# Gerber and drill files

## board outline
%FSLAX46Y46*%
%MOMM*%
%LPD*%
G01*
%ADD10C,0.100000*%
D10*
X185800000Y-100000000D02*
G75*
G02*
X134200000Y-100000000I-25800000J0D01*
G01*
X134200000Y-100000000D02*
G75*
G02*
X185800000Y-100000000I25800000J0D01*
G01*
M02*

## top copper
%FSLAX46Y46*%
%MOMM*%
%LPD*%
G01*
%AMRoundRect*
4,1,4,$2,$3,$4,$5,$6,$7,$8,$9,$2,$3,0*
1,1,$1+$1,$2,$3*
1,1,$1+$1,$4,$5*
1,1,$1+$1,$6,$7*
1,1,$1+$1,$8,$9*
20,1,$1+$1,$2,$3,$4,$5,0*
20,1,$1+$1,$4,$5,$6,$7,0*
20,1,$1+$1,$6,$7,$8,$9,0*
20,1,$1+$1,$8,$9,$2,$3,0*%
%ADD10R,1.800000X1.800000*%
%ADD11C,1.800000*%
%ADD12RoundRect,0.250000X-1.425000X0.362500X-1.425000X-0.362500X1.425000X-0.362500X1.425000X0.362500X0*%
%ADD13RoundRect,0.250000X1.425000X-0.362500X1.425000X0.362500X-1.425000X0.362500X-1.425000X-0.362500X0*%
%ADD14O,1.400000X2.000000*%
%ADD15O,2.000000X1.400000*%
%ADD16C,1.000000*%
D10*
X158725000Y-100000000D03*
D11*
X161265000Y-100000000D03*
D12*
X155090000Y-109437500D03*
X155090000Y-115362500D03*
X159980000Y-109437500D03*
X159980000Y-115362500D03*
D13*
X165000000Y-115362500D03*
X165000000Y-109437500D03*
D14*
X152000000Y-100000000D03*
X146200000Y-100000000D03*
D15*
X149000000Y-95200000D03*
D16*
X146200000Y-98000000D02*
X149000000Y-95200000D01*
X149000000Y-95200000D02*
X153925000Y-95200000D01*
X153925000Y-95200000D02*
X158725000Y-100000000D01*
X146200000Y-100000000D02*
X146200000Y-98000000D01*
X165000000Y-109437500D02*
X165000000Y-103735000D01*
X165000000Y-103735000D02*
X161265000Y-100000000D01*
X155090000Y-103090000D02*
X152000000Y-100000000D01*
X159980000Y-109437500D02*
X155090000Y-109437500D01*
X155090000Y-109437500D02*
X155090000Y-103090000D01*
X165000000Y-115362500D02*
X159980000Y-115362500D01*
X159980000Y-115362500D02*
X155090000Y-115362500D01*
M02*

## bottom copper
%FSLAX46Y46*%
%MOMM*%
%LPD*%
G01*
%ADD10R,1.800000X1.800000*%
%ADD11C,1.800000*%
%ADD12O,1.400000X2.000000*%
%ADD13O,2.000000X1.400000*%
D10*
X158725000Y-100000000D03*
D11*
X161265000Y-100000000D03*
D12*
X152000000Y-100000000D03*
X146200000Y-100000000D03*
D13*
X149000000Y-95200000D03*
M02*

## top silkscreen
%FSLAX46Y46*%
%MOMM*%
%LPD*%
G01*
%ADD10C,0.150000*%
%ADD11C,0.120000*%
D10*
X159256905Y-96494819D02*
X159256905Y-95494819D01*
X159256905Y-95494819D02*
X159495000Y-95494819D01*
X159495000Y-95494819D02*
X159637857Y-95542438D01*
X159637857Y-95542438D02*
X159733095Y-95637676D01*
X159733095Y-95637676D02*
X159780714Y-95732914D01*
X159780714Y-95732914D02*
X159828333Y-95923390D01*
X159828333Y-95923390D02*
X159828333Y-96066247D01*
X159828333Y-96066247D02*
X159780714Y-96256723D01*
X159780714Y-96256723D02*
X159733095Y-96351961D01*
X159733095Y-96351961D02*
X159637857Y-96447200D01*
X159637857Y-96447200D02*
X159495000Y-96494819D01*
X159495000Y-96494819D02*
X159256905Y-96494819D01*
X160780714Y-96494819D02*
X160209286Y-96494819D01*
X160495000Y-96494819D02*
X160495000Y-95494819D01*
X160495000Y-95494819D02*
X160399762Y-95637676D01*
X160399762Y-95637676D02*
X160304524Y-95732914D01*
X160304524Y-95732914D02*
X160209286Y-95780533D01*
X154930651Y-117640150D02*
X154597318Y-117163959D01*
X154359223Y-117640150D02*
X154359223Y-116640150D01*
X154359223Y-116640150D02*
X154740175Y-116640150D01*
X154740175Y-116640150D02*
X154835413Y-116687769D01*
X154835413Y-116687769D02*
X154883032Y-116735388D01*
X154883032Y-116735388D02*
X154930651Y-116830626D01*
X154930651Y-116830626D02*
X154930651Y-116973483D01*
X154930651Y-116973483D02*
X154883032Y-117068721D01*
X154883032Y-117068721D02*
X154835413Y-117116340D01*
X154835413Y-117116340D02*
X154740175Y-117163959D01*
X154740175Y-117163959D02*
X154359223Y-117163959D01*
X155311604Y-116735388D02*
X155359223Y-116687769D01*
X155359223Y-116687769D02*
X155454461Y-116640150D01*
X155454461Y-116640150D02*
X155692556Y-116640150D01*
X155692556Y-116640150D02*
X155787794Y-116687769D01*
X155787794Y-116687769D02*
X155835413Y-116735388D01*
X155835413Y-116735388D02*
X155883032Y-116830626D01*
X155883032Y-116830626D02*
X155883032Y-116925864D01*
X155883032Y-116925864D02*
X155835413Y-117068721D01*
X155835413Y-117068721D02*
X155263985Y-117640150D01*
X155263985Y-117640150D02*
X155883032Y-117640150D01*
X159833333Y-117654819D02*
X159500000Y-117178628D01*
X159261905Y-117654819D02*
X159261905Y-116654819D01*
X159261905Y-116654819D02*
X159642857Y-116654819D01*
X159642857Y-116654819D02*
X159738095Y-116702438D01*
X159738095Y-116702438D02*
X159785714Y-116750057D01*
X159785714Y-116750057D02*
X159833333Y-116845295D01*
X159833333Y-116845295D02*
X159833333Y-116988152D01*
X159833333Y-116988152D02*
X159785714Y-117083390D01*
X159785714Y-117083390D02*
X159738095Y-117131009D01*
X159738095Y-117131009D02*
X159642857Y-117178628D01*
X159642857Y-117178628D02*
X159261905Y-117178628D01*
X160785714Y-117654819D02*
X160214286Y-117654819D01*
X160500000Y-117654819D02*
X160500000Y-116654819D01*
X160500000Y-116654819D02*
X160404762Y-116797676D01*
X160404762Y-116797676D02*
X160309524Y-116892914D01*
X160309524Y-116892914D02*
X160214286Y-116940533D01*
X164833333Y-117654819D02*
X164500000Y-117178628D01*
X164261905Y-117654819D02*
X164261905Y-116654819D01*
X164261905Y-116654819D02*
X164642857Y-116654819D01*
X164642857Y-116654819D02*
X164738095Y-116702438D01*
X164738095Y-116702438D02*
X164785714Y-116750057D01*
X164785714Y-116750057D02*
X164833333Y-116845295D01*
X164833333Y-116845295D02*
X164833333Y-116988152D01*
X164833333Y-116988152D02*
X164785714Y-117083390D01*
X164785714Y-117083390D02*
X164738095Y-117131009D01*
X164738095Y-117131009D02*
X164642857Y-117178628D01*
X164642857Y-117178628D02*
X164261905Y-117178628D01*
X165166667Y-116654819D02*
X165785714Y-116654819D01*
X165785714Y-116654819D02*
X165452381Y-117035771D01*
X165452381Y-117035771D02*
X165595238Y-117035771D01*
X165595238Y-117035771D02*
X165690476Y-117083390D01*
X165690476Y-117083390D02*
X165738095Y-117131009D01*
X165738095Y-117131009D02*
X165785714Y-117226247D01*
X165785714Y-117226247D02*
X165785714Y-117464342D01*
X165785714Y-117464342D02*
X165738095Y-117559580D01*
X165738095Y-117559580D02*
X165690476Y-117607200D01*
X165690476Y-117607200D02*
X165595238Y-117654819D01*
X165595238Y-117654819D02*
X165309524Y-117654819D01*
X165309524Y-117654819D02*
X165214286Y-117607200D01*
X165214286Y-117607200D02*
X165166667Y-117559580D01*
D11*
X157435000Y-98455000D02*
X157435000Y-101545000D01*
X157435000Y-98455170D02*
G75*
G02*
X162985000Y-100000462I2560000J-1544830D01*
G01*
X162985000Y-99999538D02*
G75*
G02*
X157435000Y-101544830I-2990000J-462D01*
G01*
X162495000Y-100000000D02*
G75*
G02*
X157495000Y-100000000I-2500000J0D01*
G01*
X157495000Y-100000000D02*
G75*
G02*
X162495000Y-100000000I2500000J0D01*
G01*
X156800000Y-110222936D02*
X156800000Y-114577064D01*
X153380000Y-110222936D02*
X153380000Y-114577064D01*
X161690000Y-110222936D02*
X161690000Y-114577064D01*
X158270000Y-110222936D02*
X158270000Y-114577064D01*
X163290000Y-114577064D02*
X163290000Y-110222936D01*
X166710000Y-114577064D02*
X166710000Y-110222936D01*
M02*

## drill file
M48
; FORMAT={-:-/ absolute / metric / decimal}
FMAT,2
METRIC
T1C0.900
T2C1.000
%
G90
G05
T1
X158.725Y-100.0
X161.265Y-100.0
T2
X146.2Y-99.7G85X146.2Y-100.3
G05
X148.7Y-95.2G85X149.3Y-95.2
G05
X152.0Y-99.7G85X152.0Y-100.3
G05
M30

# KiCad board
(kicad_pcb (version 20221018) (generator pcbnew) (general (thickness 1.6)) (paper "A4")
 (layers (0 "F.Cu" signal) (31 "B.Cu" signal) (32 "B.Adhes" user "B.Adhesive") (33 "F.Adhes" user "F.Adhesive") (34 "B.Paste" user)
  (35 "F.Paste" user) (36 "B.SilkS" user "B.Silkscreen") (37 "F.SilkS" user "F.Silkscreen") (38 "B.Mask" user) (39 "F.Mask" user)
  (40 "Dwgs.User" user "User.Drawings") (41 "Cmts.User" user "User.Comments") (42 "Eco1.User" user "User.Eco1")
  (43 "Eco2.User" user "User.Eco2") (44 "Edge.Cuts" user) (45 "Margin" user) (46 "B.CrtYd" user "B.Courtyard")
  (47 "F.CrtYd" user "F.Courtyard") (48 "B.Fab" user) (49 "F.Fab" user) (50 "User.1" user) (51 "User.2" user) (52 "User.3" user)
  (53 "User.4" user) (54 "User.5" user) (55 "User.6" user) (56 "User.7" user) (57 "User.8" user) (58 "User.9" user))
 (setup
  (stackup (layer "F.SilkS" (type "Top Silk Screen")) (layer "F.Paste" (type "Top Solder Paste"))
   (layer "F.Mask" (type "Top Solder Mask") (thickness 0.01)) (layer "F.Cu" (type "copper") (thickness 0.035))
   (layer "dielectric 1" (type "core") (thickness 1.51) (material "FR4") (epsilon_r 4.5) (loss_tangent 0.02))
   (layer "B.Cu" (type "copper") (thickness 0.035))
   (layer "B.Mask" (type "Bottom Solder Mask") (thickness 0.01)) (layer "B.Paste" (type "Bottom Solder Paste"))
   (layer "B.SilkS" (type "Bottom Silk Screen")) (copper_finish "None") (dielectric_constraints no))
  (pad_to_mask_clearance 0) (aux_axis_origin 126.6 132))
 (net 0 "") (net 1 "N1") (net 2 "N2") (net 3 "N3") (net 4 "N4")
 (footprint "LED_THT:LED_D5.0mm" (layer "F.Cu") (at 158.725 100)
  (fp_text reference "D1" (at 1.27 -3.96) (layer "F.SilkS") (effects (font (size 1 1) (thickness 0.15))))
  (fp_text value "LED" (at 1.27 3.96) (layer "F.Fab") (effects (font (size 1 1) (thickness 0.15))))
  (fp_line (start -1.29 -1.545) (end -1.29 1.545) (stroke (width 0.12) (type solid)) (layer "F.SilkS"))
  (fp_arc (start -1.29 -1.54483) (mid 2.072002 -2.880433) (end 4.26 0.000462) (stroke (width 0.12) (type solid)) (layer "F.SilkS"))
  (fp_arc (start 4.26 -0.000462) (mid 2.072002 2.880433) (end -1.29 1.54483) (stroke (width 0.12) (type solid)) (layer "F.SilkS"))
  (fp_circle (center 1.27 0) (end 3.77 0) (stroke (width 0.12) (type solid)) (fill none) (layer "F.SilkS"))
  (pad "1" thru_hole rect (at 0 0) (size 1.8 1.8) (drill 0.9) (layers "*.Cu" "*.Mask") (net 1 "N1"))
  (pad "2" thru_hole circle (at 2.54 0) (size 1.8 1.8) (drill 0.9) (layers "*.Cu" "*.Mask") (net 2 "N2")))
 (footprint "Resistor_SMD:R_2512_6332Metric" (layer "F.Cu") (at 155.09 112.4 -90)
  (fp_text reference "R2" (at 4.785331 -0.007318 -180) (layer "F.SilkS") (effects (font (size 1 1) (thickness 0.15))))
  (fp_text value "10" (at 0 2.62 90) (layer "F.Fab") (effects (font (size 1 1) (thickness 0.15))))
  (fp_line (start -2.177064 -1.71) (end 2.177064 -1.71) (stroke (width 0.12) (type solid)) (layer "F.SilkS"))
  (fp_line (start -2.177064 1.71) (end 2.177064 1.71) (stroke (width 0.12) (type solid)) (layer "F.SilkS"))
  (pad "1" smd roundrect (at -2.9625 0 270) (size 1.225 3.35) (layers "F.Cu" "F.Paste" "F.Mask") (roundrect_rratio 0.2040816327)
   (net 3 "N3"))
  (pad "2" smd roundrect (at 2.9625 0 270) (size 1.225 3.35) (layers "F.Cu" "F.Paste" "F.Mask") (roundrect_rratio 0.2040816327) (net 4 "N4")))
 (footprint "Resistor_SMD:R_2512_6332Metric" (layer "F.Cu") (at 159.98 112.4 -90)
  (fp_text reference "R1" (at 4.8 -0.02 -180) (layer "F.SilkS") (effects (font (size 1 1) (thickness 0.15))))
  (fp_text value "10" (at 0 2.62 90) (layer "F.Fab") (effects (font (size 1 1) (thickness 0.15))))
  (fp_line (start -2.177064 -1.71) (end 2.177064 -1.71) (stroke (width 0.12) (type solid)) (layer "F.SilkS"))
  (fp_line (start -2.177064 1.71) (end 2.177064 1.71) (stroke (width 0.12) (type solid)) (layer "F.SilkS"))
  (pad "1" smd roundrect (at -2.9625 0 270) (size 1.225 3.35) (layers "F.Cu" "F.Paste" "F.Mask") (roundrect_rratio 0.2040816327)
   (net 3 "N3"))
  (pad "2" smd roundrect (at 2.9625 0 270) (size 1.225 3.35) (layers "F.Cu" "F.Paste" "F.Mask") (roundrect_rratio 0.2040816327) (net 4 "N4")))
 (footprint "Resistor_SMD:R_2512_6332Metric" (layer "F.Cu") (at 165 112.4 90)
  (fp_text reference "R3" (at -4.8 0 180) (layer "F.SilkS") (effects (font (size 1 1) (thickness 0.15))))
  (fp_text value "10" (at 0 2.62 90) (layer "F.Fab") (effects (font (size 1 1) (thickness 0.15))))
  (fp_line (start -2.177064 -1.71) (end 2.177064 -1.71) (stroke (width 0.12) (type solid)) (layer "F.SilkS"))
  (fp_line (start -2.177064 1.71) (end 2.177064 1.71) (stroke (width 0.12) (type solid)) (layer "F.SilkS"))
  (pad "1" smd roundrect (at -2.9625 0 90) (size 1.225 3.35) (layers "F.Cu" "F.Paste" "F.Mask") (roundrect_rratio 0.2040816327) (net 4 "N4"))
  (pad "2" smd roundrect (at 2.9625 0 90) (size 1.225 3.35) (layers "F.Cu" "F.Paste" "F.Mask") (roundrect_rratio 0.2040816327) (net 2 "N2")))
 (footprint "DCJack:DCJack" (layer "B.Cu") (at 146.2 100)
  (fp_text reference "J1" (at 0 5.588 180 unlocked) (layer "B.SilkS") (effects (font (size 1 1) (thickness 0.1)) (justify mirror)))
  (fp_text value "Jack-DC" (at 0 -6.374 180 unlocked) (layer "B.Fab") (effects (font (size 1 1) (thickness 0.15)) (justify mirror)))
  (pad "1" thru_hole oval (at 5.8 0) (size 1.4 2) (drill oval 1 1.6) (layers "*.Cu" "*.Mask") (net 3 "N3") (thermal_bridge_angle 45))
  (pad "2" thru_hole oval (at 0 0) (size 1.4 2) (drill oval 1 1.6) (layers "*.Cu" "*.Mask") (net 1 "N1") (thermal_bridge_angle 45))
  (pad "2" thru_hole oval (at 2.8 -4.8) (size 2 1.4) (drill oval 1.6 1) (layers "*.Cu" "*.Mask") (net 1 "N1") (thermal_bridge_angle 45)))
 (gr_circle (center 160 100) (end 185.8 100) (stroke (width 0.1) (type default)) (fill none) (layer "Edge.Cuts"))
 (segment (start 146.2 98) (end 149 95.2) (width 1) (layer "F.Cu") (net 1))
 (segment (start 149 95.2) (end 153.925 95.2) (width 1) (layer "F.Cu") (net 1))
 (segment (start 153.925 95.2) (end 158.725 100) (width 1) (layer "F.Cu") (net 1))
 (segment (start 146.2 100) (end 146.2 98) (width 1) (layer "F.Cu") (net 1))
 (segment (start 165 109.4375) (end 165 103.735) (width 1) (layer "F.Cu") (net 2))
 (segment (start 165 103.735) (end 161.265 100) (width 1) (layer "F.Cu") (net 2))
 (segment (start 155.09 103.09) (end 152 100) (width 1) (layer "F.Cu") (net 3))
 (segment (start 159.98 109.4375) (end 155.09 109.4375) (width 1) (layer "F.Cu") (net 3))
 (segment (start 155.09 109.4375) (end 155.09 103.09) (width 1) (layer "F.Cu") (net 3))
 (segment (start 165 115.3625) (end 159.98 115.3625) (width 1) (layer "F.Cu") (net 4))
 (segment (start 159.98 115.3625) (end 155.09 115.3625) (width 1) (layer "F.Cu") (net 4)))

